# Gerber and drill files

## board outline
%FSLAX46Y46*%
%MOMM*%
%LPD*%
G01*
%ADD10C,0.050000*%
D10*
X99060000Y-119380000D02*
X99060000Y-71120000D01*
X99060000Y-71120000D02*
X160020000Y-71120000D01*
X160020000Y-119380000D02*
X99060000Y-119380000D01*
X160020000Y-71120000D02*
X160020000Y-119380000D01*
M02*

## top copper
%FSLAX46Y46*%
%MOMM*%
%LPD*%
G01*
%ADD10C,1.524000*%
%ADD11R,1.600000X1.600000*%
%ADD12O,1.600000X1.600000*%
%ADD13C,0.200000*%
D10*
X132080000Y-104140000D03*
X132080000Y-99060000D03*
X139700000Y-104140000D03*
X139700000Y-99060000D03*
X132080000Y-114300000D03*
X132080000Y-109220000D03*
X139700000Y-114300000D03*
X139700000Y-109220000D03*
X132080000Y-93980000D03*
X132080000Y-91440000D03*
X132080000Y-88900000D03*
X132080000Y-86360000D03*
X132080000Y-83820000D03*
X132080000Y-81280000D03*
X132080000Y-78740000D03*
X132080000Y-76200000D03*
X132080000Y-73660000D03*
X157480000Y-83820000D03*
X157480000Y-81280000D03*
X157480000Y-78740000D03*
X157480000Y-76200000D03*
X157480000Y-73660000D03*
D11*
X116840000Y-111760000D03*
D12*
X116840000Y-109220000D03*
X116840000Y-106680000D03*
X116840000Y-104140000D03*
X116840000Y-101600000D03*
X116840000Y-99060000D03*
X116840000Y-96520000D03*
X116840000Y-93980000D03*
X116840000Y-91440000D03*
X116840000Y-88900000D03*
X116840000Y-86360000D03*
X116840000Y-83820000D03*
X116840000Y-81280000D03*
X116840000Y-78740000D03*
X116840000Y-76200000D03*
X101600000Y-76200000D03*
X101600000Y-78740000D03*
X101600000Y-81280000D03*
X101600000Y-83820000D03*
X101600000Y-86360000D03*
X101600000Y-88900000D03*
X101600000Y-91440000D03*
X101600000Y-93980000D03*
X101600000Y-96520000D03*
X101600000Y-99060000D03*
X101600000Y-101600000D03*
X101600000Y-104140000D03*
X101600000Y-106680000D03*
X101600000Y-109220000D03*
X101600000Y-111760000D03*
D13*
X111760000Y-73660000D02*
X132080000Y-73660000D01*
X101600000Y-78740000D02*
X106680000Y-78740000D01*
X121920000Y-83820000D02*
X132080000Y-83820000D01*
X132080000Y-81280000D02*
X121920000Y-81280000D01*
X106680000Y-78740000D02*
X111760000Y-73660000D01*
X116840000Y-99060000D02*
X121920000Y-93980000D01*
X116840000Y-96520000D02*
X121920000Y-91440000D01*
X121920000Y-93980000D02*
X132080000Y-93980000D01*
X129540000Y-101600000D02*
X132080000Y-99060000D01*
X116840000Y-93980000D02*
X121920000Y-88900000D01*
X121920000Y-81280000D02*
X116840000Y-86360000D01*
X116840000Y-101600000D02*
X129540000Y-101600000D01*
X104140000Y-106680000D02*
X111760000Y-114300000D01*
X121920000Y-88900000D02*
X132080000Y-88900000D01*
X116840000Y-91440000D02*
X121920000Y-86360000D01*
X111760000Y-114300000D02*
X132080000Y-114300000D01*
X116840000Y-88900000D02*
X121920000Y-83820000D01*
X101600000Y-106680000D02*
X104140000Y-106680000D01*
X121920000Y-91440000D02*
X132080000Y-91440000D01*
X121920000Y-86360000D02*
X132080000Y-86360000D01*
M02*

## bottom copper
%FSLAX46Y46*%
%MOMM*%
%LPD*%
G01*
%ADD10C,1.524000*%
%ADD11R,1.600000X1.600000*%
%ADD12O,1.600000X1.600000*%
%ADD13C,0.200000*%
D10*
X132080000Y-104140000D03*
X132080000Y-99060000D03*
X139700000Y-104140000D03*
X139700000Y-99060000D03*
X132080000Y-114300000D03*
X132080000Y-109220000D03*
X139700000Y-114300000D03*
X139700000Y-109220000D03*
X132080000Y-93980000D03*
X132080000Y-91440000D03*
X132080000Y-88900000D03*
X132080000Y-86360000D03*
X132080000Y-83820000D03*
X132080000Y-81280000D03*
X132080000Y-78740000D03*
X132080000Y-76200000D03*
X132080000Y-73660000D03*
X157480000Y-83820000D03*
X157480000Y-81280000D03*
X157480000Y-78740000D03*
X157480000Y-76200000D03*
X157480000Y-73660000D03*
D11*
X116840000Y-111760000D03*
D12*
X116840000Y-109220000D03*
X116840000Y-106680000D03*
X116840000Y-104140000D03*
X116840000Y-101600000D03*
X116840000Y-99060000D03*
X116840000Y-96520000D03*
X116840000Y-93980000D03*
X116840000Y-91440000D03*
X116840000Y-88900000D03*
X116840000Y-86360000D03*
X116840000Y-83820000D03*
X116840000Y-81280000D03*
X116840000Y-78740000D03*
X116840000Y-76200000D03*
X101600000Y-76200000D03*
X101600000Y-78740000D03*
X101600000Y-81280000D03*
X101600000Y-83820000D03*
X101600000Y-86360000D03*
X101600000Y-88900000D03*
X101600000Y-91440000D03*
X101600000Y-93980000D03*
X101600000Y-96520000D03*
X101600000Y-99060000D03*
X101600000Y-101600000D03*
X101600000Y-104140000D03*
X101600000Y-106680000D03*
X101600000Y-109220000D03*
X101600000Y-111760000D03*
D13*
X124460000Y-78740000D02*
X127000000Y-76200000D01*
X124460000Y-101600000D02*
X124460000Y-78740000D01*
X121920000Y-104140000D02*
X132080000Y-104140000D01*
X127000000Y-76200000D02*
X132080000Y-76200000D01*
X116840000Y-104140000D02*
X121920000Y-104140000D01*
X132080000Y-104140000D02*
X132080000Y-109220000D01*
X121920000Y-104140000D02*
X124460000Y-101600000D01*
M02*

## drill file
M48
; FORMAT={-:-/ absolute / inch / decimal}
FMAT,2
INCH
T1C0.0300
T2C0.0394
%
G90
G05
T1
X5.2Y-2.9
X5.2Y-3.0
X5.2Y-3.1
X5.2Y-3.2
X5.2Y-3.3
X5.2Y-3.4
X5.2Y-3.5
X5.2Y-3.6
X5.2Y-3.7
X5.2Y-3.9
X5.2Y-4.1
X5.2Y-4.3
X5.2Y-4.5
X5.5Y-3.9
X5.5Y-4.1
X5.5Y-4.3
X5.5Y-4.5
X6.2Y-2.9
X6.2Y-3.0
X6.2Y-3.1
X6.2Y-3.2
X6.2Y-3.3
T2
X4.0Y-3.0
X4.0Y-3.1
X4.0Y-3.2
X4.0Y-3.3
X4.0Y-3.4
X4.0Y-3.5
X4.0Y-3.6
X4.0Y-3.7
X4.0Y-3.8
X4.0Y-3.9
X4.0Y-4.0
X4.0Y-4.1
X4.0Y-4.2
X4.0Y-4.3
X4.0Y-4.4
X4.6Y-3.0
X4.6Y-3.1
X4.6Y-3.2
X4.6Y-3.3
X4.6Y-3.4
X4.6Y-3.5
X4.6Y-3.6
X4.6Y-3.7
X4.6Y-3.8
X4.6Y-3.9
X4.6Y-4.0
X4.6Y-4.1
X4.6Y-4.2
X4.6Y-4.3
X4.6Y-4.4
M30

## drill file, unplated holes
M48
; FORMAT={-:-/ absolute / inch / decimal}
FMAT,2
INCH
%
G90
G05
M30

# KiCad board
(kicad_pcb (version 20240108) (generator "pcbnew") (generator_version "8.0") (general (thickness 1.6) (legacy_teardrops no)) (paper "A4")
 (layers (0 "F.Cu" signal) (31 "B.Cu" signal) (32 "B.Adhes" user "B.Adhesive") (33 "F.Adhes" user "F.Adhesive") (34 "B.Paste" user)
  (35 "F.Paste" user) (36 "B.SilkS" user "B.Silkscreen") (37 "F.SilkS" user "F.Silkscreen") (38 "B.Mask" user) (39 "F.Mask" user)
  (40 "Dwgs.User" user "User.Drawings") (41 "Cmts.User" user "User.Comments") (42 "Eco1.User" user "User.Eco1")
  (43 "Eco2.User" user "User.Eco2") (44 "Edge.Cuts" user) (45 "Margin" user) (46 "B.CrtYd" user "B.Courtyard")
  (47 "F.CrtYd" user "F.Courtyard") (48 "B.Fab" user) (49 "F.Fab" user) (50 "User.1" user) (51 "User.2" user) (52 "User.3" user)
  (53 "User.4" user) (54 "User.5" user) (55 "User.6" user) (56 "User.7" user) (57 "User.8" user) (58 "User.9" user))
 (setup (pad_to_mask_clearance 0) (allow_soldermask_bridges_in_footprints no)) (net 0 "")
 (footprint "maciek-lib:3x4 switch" (layer "F.Cu") (at 134.62 101.6 90)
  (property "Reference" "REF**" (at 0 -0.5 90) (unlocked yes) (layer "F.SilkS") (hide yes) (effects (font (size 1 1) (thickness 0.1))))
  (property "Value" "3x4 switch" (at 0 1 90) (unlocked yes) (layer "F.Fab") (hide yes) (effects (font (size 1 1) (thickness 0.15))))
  (pad "1" thru_hole circle (at -2.54 -2.54 90) (size 1.524 1.524) (drill 0.762) (layers "*.Cu" "*.Mask") (remove_unused_layers no))
  (pad "2" thru_hole circle (at 2.54 -2.54 90) (size 1.524 1.524) (drill 0.762) (layers "*.Cu" "*.Mask") (remove_unused_layers no))
  (pad "3" thru_hole circle (at -2.54 5.08 90) (size 1.524 1.524) (drill 0.762) (layers "*.Cu" "*.Mask") (remove_unused_layers no))
  (pad "4" thru_hole circle (at 2.54 5.08 90) (size 1.524 1.524) (drill 0.762) (layers "*.Cu" "*.Mask") (remove_unused_layers no)))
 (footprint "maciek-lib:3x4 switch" (layer "F.Cu") (at 134.62 111.76 90)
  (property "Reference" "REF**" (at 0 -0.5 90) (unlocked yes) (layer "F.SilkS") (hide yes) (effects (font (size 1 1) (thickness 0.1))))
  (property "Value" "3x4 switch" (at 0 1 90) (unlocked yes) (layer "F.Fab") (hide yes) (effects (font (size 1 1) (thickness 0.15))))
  (pad "1" thru_hole circle (at -2.54 -2.54 90) (size 1.524 1.524) (drill 0.762) (layers "*.Cu" "*.Mask") (remove_unused_layers no))
  (pad "2" thru_hole circle (at 2.54 -2.54 90) (size 1.524 1.524) (drill 0.762) (layers "*.Cu" "*.Mask") (remove_unused_layers no))
  (pad "3" thru_hole circle (at -2.54 5.08 90) (size 1.524 1.524) (drill 0.762) (layers "*.Cu" "*.Mask") (remove_unused_layers no))
  (pad "4" thru_hole circle (at 2.54 5.08 90) (size 1.524 1.524) (drill 0.762) (layers "*.Cu" "*.Mask") (remove_unused_layers no)))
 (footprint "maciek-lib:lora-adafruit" (layer "F.Cu") (at 144.78 83.82 90)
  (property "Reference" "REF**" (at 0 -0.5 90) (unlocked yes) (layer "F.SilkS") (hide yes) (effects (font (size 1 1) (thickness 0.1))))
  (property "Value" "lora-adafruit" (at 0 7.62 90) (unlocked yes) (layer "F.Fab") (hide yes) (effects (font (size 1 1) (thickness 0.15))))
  (pad "1" thru_hole circle (at -10.16 -12.7 90) (size 1.524 1.524) (drill 0.762) (layers "*.Cu" "*.Mask") (remove_unused_layers no))
  (pad "2" thru_hole circle (at -7.62 -12.7 90) (size 1.524 1.524) (drill 0.762) (layers "*.Cu" "*.Mask") (remove_unused_layers no))
  (pad "3" thru_hole circle (at -5.08 -12.7 90) (size 1.524 1.524) (drill 0.762) (layers "*.Cu" "*.Mask") (remove_unused_layers no))
  (pad "4" thru_hole circle (at -2.54 -12.7 90) (size 1.524 1.524) (drill 0.762) (layers "*.Cu" "*.Mask") (remove_unused_layers no))
  (pad "5" thru_hole circle (at 0 -12.7 90) (size 1.524 1.524) (drill 0.762) (layers "*.Cu" "*.Mask") (remove_unused_layers no))
  (pad "6" thru_hole circle (at 2.54 -12.7 90) (size 1.524 1.524) (drill 0.762) (layers "*.Cu" "*.Mask") (remove_unused_layers no))
  (pad "7" thru_hole circle (at 5.08 -12.7 90) (size 1.524 1.524) (drill 0.762) (layers "*.Cu" "*.Mask") (remove_unused_layers no))
  (pad "8" thru_hole circle (at 7.62 -12.7 90) (size 1.524 1.524) (drill 0.762) (layers "*.Cu" "*.Mask") (remove_unused_layers no))
  (pad "9" thru_hole circle (at 10.16 -12.7 90) (size 1.524 1.524) (drill 0.762) (layers "*.Cu" "*.Mask") (remove_unused_layers no))
  (pad "10" thru_hole circle (at 0 12.7 90) (size 1.524 1.524) (drill 0.762) (layers "*.Cu" "*.Mask") (remove_unused_layers no))
  (pad "11" thru_hole circle (at 2.54 12.7 90) (size 1.524 1.524) (drill 0.762) (layers "*.Cu" "*.Mask") (remove_unused_layers no))
  (pad "12" thru_hole circle (at 5.08 12.7 90) (size 1.524 1.524) (drill 0.762) (layers "*.Cu" "*.Mask") (remove_unused_layers no))
  (pad "13" thru_hole circle (at 7.62 12.7 90) (size 1.524 1.524) (drill 0.762) (layers "*.Cu" "*.Mask") (remove_unused_layers no))
  (pad "14" thru_hole circle (at 10.16 12.7 90) (size 1.524 1.524) (drill 0.762) (layers "*.Cu" "*.Mask") (remove_unused_layers no)))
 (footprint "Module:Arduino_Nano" (layer "F.Cu") (at 116.84 111.76 180)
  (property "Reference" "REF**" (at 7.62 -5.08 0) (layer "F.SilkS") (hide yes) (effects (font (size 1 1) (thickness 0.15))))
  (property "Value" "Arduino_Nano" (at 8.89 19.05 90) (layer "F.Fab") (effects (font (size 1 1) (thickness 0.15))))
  (pad "1" thru_hole rect (at 0 0 180) (size 1.6 1.6) (drill 1) (layers "*.Cu" "*.Mask") (remove_unused_layers no))
  (pad "2" thru_hole oval (at 0 2.54 180) (size 1.6 1.6) (drill 1) (layers "*.Cu" "*.Mask") (remove_unused_layers no))
  (pad "3" thru_hole oval (at 0 5.08 180) (size 1.6 1.6) (drill 1) (layers "*.Cu" "*.Mask") (remove_unused_layers no))
  (pad "4" thru_hole oval (at 0 7.62 180) (size 1.6 1.6) (drill 1) (layers "*.Cu" "*.Mask") (remove_unused_layers no))
  (pad "5" thru_hole oval (at 0 10.16 180) (size 1.6 1.6) (drill 1) (layers "*.Cu" "*.Mask") (remove_unused_layers no))
  (pad "6" thru_hole oval (at 0 12.7 180) (size 1.6 1.6) (drill 1) (layers "*.Cu" "*.Mask") (remove_unused_layers no))
  (pad "7" thru_hole oval (at 0 15.24 180) (size 1.6 1.6) (drill 1) (layers "*.Cu" "*.Mask") (remove_unused_layers no))
  (pad "8" thru_hole oval (at 0 17.78 180) (size 1.6 1.6) (drill 1) (layers "*.Cu" "*.Mask") (remove_unused_layers no))
  (pad "9" thru_hole oval (at 0 20.32 180) (size 1.6 1.6) (drill 1) (layers "*.Cu" "*.Mask") (remove_unused_layers no))
  (pad "10" thru_hole oval (at 0 22.86 180) (size 1.6 1.6) (drill 1) (layers "*.Cu" "*.Mask") (remove_unused_layers no))
  (pad "11" thru_hole oval (at 0 25.4 180) (size 1.6 1.6) (drill 1) (layers "*.Cu" "*.Mask") (remove_unused_layers no))
  (pad "12" thru_hole oval (at 0 27.94 180) (size 1.6 1.6) (drill 1) (layers "*.Cu" "*.Mask") (remove_unused_layers no))
  (pad "13" thru_hole oval (at 0 30.48 180) (size 1.6 1.6) (drill 1) (layers "*.Cu" "*.Mask") (remove_unused_layers no))
  (pad "14" thru_hole oval (at 0 33.02 180) (size 1.6 1.6) (drill 1) (layers "*.Cu" "*.Mask") (remove_unused_layers no))
  (pad "15" thru_hole oval (at 0 35.56 180) (size 1.6 1.6) (drill 1) (layers "*.Cu" "*.Mask") (remove_unused_layers no))
  (pad "16" thru_hole oval (at 15.24 35.56 180) (size 1.6 1.6) (drill 1) (layers "*.Cu" "*.Mask") (remove_unused_layers no))
  (pad "17" thru_hole oval (at 15.24 33.02 180) (size 1.6 1.6) (drill 1) (layers "*.Cu" "*.Mask") (remove_unused_layers no))
  (pad "18" thru_hole oval (at 15.24 30.48 180) (size 1.6 1.6) (drill 1) (layers "*.Cu" "*.Mask") (remove_unused_layers no))
  (pad "19" thru_hole oval (at 15.24 27.94 180) (size 1.6 1.6) (drill 1) (layers "*.Cu" "*.Mask") (remove_unused_layers no))
  (pad "20" thru_hole oval (at 15.24 25.4 180) (size 1.6 1.6) (drill 1) (layers "*.Cu" "*.Mask") (remove_unused_layers no))
  (pad "21" thru_hole oval (at 15.24 22.86 180) (size 1.6 1.6) (drill 1) (layers "*.Cu" "*.Mask") (remove_unused_layers no))
  (pad "22" thru_hole oval (at 15.24 20.32 180) (size 1.6 1.6) (drill 1) (layers "*.Cu" "*.Mask") (remove_unused_layers no))
  (pad "23" thru_hole oval (at 15.24 17.78 180) (size 1.6 1.6) (drill 1) (layers "*.Cu" "*.Mask") (remove_unused_layers no))
  (pad "24" thru_hole oval (at 15.24 15.24 180) (size 1.6 1.6) (drill 1) (layers "*.Cu" "*.Mask") (remove_unused_layers no))
  (pad "25" thru_hole oval (at 15.24 12.7 180) (size 1.6 1.6) (drill 1) (layers "*.Cu" "*.Mask") (remove_unused_layers no))
  (pad "26" thru_hole oval (at 15.24 10.16 180) (size 1.6 1.6) (drill 1) (layers "*.Cu" "*.Mask") (remove_unused_layers no))
  (pad "27" thru_hole oval (at 15.24 7.62 180) (size 1.6 1.6) (drill 1) (layers "*.Cu" "*.Mask") (remove_unused_layers no))
  (pad "28" thru_hole oval (at 15.24 5.08 180) (size 1.6 1.6) (drill 1) (layers "*.Cu" "*.Mask") (remove_unused_layers no))
  (pad "29" thru_hole oval (at 15.24 2.54 180) (size 1.6 1.6) (drill 1) (layers "*.Cu" "*.Mask") (remove_unused_layers no))
  (pad "30" thru_hole oval (at 15.24 0 180) (size 1.6 1.6) (drill 1) (layers "*.Cu" "*.Mask") (remove_unused_layers no)))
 (gr_line (start 99.06 119.38) (end 99.06 71.12) (stroke (width 0.05) (type default)) (layer "Edge.Cuts"))
 (gr_line (start 99.06 71.12) (end 160.02 71.12) (stroke (width 0.05) (type default)) (layer "Edge.Cuts"))
 (gr_line (start 160.02 119.38) (end 99.06 119.38) (stroke (width 0.05) (type default)) (layer "Edge.Cuts"))
 (gr_line (start 160.02 71.12) (end 160.02 119.38) (stroke (width 0.05) (type default)) (layer "Edge.Cuts"))
 (segment (start 111.76 73.66) (end 132.08 73.66) (width 0.2) (layer "F.Cu") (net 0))
 (segment (start 101.6 78.74) (end 106.68 78.74) (width 0.2) (layer "F.Cu") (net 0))
 (segment (start 121.92 83.82) (end 132.08 83.82) (width 0.2) (layer "F.Cu") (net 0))
 (segment (start 132.08 81.28) (end 121.92 81.28) (width 0.2) (layer "F.Cu") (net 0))
 (segment (start 106.68 78.74) (end 111.76 73.66) (width 0.2) (layer "F.Cu") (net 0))
 (segment (start 116.84 99.06) (end 121.92 93.98) (width 0.2) (layer "F.Cu") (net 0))
 (segment (start 116.84 96.52) (end 121.92 91.44) (width 0.2) (layer "F.Cu") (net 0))
 (segment (start 121.92 93.98) (end 132.08 93.98) (width 0.2) (layer "F.Cu") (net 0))
 (segment (start 129.54 101.6) (end 132.08 99.06) (width 0.2) (layer "F.Cu") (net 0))
 (segment (start 116.84 93.98) (end 121.92 88.9) (width 0.2) (layer "F.Cu") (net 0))
 (segment (start 121.92 81.28) (end 116.84 86.36) (width 0.2) (layer "F.Cu") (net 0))
 (segment (start 116.84 101.6) (end 129.54 101.6) (width 0.2) (layer "F.Cu") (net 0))
 (segment (start 104.14 106.68) (end 111.76 114.3) (width 0.2) (layer "F.Cu") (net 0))
 (segment (start 121.92 88.9) (end 132.08 88.9) (width 0.2) (layer "F.Cu") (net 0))
 (segment (start 116.84 91.44) (end 121.92 86.36) (width 0.2) (layer "F.Cu") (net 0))
 (segment (start 111.76 114.3) (end 132.08 114.3) (width 0.2) (layer "F.Cu") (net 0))
 (segment (start 116.84 88.9) (end 121.92 83.82) (width 0.2) (layer "F.Cu") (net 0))
 (segment (start 101.6 106.68) (end 104.14 106.68) (width 0.2) (layer "F.Cu") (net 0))
 (segment (start 121.92 91.44) (end 132.08 91.44) (width 0.2) (layer "F.Cu") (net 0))
 (segment (start 121.92 86.36) (end 132.08 86.36) (width 0.2) (layer "F.Cu") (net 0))
 (segment (start 124.46 78.74) (end 127 76.2) (width 0.2) (layer "B.Cu") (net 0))
 (segment (start 124.46 101.6) (end 124.46 78.74) (width 0.2) (layer "B.Cu") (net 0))
 (segment (start 121.92 104.14) (end 132.08 104.14) (width 0.2) (layer "B.Cu") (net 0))
 (segment (start 127 76.2) (end 132.08 76.2) (width 0.2) (layer "B.Cu") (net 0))
 (segment (start 116.84 104.14) (end 121.92 104.14) (width 0.2) (layer "B.Cu") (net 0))
 (segment (start 132.08 104.14) (end 132.08 109.22) (width 0.2) (layer "B.Cu") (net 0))
 (segment (start 121.92 104.14) (end 124.46 101.6) (width 0.2) (layer "B.Cu") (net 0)))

